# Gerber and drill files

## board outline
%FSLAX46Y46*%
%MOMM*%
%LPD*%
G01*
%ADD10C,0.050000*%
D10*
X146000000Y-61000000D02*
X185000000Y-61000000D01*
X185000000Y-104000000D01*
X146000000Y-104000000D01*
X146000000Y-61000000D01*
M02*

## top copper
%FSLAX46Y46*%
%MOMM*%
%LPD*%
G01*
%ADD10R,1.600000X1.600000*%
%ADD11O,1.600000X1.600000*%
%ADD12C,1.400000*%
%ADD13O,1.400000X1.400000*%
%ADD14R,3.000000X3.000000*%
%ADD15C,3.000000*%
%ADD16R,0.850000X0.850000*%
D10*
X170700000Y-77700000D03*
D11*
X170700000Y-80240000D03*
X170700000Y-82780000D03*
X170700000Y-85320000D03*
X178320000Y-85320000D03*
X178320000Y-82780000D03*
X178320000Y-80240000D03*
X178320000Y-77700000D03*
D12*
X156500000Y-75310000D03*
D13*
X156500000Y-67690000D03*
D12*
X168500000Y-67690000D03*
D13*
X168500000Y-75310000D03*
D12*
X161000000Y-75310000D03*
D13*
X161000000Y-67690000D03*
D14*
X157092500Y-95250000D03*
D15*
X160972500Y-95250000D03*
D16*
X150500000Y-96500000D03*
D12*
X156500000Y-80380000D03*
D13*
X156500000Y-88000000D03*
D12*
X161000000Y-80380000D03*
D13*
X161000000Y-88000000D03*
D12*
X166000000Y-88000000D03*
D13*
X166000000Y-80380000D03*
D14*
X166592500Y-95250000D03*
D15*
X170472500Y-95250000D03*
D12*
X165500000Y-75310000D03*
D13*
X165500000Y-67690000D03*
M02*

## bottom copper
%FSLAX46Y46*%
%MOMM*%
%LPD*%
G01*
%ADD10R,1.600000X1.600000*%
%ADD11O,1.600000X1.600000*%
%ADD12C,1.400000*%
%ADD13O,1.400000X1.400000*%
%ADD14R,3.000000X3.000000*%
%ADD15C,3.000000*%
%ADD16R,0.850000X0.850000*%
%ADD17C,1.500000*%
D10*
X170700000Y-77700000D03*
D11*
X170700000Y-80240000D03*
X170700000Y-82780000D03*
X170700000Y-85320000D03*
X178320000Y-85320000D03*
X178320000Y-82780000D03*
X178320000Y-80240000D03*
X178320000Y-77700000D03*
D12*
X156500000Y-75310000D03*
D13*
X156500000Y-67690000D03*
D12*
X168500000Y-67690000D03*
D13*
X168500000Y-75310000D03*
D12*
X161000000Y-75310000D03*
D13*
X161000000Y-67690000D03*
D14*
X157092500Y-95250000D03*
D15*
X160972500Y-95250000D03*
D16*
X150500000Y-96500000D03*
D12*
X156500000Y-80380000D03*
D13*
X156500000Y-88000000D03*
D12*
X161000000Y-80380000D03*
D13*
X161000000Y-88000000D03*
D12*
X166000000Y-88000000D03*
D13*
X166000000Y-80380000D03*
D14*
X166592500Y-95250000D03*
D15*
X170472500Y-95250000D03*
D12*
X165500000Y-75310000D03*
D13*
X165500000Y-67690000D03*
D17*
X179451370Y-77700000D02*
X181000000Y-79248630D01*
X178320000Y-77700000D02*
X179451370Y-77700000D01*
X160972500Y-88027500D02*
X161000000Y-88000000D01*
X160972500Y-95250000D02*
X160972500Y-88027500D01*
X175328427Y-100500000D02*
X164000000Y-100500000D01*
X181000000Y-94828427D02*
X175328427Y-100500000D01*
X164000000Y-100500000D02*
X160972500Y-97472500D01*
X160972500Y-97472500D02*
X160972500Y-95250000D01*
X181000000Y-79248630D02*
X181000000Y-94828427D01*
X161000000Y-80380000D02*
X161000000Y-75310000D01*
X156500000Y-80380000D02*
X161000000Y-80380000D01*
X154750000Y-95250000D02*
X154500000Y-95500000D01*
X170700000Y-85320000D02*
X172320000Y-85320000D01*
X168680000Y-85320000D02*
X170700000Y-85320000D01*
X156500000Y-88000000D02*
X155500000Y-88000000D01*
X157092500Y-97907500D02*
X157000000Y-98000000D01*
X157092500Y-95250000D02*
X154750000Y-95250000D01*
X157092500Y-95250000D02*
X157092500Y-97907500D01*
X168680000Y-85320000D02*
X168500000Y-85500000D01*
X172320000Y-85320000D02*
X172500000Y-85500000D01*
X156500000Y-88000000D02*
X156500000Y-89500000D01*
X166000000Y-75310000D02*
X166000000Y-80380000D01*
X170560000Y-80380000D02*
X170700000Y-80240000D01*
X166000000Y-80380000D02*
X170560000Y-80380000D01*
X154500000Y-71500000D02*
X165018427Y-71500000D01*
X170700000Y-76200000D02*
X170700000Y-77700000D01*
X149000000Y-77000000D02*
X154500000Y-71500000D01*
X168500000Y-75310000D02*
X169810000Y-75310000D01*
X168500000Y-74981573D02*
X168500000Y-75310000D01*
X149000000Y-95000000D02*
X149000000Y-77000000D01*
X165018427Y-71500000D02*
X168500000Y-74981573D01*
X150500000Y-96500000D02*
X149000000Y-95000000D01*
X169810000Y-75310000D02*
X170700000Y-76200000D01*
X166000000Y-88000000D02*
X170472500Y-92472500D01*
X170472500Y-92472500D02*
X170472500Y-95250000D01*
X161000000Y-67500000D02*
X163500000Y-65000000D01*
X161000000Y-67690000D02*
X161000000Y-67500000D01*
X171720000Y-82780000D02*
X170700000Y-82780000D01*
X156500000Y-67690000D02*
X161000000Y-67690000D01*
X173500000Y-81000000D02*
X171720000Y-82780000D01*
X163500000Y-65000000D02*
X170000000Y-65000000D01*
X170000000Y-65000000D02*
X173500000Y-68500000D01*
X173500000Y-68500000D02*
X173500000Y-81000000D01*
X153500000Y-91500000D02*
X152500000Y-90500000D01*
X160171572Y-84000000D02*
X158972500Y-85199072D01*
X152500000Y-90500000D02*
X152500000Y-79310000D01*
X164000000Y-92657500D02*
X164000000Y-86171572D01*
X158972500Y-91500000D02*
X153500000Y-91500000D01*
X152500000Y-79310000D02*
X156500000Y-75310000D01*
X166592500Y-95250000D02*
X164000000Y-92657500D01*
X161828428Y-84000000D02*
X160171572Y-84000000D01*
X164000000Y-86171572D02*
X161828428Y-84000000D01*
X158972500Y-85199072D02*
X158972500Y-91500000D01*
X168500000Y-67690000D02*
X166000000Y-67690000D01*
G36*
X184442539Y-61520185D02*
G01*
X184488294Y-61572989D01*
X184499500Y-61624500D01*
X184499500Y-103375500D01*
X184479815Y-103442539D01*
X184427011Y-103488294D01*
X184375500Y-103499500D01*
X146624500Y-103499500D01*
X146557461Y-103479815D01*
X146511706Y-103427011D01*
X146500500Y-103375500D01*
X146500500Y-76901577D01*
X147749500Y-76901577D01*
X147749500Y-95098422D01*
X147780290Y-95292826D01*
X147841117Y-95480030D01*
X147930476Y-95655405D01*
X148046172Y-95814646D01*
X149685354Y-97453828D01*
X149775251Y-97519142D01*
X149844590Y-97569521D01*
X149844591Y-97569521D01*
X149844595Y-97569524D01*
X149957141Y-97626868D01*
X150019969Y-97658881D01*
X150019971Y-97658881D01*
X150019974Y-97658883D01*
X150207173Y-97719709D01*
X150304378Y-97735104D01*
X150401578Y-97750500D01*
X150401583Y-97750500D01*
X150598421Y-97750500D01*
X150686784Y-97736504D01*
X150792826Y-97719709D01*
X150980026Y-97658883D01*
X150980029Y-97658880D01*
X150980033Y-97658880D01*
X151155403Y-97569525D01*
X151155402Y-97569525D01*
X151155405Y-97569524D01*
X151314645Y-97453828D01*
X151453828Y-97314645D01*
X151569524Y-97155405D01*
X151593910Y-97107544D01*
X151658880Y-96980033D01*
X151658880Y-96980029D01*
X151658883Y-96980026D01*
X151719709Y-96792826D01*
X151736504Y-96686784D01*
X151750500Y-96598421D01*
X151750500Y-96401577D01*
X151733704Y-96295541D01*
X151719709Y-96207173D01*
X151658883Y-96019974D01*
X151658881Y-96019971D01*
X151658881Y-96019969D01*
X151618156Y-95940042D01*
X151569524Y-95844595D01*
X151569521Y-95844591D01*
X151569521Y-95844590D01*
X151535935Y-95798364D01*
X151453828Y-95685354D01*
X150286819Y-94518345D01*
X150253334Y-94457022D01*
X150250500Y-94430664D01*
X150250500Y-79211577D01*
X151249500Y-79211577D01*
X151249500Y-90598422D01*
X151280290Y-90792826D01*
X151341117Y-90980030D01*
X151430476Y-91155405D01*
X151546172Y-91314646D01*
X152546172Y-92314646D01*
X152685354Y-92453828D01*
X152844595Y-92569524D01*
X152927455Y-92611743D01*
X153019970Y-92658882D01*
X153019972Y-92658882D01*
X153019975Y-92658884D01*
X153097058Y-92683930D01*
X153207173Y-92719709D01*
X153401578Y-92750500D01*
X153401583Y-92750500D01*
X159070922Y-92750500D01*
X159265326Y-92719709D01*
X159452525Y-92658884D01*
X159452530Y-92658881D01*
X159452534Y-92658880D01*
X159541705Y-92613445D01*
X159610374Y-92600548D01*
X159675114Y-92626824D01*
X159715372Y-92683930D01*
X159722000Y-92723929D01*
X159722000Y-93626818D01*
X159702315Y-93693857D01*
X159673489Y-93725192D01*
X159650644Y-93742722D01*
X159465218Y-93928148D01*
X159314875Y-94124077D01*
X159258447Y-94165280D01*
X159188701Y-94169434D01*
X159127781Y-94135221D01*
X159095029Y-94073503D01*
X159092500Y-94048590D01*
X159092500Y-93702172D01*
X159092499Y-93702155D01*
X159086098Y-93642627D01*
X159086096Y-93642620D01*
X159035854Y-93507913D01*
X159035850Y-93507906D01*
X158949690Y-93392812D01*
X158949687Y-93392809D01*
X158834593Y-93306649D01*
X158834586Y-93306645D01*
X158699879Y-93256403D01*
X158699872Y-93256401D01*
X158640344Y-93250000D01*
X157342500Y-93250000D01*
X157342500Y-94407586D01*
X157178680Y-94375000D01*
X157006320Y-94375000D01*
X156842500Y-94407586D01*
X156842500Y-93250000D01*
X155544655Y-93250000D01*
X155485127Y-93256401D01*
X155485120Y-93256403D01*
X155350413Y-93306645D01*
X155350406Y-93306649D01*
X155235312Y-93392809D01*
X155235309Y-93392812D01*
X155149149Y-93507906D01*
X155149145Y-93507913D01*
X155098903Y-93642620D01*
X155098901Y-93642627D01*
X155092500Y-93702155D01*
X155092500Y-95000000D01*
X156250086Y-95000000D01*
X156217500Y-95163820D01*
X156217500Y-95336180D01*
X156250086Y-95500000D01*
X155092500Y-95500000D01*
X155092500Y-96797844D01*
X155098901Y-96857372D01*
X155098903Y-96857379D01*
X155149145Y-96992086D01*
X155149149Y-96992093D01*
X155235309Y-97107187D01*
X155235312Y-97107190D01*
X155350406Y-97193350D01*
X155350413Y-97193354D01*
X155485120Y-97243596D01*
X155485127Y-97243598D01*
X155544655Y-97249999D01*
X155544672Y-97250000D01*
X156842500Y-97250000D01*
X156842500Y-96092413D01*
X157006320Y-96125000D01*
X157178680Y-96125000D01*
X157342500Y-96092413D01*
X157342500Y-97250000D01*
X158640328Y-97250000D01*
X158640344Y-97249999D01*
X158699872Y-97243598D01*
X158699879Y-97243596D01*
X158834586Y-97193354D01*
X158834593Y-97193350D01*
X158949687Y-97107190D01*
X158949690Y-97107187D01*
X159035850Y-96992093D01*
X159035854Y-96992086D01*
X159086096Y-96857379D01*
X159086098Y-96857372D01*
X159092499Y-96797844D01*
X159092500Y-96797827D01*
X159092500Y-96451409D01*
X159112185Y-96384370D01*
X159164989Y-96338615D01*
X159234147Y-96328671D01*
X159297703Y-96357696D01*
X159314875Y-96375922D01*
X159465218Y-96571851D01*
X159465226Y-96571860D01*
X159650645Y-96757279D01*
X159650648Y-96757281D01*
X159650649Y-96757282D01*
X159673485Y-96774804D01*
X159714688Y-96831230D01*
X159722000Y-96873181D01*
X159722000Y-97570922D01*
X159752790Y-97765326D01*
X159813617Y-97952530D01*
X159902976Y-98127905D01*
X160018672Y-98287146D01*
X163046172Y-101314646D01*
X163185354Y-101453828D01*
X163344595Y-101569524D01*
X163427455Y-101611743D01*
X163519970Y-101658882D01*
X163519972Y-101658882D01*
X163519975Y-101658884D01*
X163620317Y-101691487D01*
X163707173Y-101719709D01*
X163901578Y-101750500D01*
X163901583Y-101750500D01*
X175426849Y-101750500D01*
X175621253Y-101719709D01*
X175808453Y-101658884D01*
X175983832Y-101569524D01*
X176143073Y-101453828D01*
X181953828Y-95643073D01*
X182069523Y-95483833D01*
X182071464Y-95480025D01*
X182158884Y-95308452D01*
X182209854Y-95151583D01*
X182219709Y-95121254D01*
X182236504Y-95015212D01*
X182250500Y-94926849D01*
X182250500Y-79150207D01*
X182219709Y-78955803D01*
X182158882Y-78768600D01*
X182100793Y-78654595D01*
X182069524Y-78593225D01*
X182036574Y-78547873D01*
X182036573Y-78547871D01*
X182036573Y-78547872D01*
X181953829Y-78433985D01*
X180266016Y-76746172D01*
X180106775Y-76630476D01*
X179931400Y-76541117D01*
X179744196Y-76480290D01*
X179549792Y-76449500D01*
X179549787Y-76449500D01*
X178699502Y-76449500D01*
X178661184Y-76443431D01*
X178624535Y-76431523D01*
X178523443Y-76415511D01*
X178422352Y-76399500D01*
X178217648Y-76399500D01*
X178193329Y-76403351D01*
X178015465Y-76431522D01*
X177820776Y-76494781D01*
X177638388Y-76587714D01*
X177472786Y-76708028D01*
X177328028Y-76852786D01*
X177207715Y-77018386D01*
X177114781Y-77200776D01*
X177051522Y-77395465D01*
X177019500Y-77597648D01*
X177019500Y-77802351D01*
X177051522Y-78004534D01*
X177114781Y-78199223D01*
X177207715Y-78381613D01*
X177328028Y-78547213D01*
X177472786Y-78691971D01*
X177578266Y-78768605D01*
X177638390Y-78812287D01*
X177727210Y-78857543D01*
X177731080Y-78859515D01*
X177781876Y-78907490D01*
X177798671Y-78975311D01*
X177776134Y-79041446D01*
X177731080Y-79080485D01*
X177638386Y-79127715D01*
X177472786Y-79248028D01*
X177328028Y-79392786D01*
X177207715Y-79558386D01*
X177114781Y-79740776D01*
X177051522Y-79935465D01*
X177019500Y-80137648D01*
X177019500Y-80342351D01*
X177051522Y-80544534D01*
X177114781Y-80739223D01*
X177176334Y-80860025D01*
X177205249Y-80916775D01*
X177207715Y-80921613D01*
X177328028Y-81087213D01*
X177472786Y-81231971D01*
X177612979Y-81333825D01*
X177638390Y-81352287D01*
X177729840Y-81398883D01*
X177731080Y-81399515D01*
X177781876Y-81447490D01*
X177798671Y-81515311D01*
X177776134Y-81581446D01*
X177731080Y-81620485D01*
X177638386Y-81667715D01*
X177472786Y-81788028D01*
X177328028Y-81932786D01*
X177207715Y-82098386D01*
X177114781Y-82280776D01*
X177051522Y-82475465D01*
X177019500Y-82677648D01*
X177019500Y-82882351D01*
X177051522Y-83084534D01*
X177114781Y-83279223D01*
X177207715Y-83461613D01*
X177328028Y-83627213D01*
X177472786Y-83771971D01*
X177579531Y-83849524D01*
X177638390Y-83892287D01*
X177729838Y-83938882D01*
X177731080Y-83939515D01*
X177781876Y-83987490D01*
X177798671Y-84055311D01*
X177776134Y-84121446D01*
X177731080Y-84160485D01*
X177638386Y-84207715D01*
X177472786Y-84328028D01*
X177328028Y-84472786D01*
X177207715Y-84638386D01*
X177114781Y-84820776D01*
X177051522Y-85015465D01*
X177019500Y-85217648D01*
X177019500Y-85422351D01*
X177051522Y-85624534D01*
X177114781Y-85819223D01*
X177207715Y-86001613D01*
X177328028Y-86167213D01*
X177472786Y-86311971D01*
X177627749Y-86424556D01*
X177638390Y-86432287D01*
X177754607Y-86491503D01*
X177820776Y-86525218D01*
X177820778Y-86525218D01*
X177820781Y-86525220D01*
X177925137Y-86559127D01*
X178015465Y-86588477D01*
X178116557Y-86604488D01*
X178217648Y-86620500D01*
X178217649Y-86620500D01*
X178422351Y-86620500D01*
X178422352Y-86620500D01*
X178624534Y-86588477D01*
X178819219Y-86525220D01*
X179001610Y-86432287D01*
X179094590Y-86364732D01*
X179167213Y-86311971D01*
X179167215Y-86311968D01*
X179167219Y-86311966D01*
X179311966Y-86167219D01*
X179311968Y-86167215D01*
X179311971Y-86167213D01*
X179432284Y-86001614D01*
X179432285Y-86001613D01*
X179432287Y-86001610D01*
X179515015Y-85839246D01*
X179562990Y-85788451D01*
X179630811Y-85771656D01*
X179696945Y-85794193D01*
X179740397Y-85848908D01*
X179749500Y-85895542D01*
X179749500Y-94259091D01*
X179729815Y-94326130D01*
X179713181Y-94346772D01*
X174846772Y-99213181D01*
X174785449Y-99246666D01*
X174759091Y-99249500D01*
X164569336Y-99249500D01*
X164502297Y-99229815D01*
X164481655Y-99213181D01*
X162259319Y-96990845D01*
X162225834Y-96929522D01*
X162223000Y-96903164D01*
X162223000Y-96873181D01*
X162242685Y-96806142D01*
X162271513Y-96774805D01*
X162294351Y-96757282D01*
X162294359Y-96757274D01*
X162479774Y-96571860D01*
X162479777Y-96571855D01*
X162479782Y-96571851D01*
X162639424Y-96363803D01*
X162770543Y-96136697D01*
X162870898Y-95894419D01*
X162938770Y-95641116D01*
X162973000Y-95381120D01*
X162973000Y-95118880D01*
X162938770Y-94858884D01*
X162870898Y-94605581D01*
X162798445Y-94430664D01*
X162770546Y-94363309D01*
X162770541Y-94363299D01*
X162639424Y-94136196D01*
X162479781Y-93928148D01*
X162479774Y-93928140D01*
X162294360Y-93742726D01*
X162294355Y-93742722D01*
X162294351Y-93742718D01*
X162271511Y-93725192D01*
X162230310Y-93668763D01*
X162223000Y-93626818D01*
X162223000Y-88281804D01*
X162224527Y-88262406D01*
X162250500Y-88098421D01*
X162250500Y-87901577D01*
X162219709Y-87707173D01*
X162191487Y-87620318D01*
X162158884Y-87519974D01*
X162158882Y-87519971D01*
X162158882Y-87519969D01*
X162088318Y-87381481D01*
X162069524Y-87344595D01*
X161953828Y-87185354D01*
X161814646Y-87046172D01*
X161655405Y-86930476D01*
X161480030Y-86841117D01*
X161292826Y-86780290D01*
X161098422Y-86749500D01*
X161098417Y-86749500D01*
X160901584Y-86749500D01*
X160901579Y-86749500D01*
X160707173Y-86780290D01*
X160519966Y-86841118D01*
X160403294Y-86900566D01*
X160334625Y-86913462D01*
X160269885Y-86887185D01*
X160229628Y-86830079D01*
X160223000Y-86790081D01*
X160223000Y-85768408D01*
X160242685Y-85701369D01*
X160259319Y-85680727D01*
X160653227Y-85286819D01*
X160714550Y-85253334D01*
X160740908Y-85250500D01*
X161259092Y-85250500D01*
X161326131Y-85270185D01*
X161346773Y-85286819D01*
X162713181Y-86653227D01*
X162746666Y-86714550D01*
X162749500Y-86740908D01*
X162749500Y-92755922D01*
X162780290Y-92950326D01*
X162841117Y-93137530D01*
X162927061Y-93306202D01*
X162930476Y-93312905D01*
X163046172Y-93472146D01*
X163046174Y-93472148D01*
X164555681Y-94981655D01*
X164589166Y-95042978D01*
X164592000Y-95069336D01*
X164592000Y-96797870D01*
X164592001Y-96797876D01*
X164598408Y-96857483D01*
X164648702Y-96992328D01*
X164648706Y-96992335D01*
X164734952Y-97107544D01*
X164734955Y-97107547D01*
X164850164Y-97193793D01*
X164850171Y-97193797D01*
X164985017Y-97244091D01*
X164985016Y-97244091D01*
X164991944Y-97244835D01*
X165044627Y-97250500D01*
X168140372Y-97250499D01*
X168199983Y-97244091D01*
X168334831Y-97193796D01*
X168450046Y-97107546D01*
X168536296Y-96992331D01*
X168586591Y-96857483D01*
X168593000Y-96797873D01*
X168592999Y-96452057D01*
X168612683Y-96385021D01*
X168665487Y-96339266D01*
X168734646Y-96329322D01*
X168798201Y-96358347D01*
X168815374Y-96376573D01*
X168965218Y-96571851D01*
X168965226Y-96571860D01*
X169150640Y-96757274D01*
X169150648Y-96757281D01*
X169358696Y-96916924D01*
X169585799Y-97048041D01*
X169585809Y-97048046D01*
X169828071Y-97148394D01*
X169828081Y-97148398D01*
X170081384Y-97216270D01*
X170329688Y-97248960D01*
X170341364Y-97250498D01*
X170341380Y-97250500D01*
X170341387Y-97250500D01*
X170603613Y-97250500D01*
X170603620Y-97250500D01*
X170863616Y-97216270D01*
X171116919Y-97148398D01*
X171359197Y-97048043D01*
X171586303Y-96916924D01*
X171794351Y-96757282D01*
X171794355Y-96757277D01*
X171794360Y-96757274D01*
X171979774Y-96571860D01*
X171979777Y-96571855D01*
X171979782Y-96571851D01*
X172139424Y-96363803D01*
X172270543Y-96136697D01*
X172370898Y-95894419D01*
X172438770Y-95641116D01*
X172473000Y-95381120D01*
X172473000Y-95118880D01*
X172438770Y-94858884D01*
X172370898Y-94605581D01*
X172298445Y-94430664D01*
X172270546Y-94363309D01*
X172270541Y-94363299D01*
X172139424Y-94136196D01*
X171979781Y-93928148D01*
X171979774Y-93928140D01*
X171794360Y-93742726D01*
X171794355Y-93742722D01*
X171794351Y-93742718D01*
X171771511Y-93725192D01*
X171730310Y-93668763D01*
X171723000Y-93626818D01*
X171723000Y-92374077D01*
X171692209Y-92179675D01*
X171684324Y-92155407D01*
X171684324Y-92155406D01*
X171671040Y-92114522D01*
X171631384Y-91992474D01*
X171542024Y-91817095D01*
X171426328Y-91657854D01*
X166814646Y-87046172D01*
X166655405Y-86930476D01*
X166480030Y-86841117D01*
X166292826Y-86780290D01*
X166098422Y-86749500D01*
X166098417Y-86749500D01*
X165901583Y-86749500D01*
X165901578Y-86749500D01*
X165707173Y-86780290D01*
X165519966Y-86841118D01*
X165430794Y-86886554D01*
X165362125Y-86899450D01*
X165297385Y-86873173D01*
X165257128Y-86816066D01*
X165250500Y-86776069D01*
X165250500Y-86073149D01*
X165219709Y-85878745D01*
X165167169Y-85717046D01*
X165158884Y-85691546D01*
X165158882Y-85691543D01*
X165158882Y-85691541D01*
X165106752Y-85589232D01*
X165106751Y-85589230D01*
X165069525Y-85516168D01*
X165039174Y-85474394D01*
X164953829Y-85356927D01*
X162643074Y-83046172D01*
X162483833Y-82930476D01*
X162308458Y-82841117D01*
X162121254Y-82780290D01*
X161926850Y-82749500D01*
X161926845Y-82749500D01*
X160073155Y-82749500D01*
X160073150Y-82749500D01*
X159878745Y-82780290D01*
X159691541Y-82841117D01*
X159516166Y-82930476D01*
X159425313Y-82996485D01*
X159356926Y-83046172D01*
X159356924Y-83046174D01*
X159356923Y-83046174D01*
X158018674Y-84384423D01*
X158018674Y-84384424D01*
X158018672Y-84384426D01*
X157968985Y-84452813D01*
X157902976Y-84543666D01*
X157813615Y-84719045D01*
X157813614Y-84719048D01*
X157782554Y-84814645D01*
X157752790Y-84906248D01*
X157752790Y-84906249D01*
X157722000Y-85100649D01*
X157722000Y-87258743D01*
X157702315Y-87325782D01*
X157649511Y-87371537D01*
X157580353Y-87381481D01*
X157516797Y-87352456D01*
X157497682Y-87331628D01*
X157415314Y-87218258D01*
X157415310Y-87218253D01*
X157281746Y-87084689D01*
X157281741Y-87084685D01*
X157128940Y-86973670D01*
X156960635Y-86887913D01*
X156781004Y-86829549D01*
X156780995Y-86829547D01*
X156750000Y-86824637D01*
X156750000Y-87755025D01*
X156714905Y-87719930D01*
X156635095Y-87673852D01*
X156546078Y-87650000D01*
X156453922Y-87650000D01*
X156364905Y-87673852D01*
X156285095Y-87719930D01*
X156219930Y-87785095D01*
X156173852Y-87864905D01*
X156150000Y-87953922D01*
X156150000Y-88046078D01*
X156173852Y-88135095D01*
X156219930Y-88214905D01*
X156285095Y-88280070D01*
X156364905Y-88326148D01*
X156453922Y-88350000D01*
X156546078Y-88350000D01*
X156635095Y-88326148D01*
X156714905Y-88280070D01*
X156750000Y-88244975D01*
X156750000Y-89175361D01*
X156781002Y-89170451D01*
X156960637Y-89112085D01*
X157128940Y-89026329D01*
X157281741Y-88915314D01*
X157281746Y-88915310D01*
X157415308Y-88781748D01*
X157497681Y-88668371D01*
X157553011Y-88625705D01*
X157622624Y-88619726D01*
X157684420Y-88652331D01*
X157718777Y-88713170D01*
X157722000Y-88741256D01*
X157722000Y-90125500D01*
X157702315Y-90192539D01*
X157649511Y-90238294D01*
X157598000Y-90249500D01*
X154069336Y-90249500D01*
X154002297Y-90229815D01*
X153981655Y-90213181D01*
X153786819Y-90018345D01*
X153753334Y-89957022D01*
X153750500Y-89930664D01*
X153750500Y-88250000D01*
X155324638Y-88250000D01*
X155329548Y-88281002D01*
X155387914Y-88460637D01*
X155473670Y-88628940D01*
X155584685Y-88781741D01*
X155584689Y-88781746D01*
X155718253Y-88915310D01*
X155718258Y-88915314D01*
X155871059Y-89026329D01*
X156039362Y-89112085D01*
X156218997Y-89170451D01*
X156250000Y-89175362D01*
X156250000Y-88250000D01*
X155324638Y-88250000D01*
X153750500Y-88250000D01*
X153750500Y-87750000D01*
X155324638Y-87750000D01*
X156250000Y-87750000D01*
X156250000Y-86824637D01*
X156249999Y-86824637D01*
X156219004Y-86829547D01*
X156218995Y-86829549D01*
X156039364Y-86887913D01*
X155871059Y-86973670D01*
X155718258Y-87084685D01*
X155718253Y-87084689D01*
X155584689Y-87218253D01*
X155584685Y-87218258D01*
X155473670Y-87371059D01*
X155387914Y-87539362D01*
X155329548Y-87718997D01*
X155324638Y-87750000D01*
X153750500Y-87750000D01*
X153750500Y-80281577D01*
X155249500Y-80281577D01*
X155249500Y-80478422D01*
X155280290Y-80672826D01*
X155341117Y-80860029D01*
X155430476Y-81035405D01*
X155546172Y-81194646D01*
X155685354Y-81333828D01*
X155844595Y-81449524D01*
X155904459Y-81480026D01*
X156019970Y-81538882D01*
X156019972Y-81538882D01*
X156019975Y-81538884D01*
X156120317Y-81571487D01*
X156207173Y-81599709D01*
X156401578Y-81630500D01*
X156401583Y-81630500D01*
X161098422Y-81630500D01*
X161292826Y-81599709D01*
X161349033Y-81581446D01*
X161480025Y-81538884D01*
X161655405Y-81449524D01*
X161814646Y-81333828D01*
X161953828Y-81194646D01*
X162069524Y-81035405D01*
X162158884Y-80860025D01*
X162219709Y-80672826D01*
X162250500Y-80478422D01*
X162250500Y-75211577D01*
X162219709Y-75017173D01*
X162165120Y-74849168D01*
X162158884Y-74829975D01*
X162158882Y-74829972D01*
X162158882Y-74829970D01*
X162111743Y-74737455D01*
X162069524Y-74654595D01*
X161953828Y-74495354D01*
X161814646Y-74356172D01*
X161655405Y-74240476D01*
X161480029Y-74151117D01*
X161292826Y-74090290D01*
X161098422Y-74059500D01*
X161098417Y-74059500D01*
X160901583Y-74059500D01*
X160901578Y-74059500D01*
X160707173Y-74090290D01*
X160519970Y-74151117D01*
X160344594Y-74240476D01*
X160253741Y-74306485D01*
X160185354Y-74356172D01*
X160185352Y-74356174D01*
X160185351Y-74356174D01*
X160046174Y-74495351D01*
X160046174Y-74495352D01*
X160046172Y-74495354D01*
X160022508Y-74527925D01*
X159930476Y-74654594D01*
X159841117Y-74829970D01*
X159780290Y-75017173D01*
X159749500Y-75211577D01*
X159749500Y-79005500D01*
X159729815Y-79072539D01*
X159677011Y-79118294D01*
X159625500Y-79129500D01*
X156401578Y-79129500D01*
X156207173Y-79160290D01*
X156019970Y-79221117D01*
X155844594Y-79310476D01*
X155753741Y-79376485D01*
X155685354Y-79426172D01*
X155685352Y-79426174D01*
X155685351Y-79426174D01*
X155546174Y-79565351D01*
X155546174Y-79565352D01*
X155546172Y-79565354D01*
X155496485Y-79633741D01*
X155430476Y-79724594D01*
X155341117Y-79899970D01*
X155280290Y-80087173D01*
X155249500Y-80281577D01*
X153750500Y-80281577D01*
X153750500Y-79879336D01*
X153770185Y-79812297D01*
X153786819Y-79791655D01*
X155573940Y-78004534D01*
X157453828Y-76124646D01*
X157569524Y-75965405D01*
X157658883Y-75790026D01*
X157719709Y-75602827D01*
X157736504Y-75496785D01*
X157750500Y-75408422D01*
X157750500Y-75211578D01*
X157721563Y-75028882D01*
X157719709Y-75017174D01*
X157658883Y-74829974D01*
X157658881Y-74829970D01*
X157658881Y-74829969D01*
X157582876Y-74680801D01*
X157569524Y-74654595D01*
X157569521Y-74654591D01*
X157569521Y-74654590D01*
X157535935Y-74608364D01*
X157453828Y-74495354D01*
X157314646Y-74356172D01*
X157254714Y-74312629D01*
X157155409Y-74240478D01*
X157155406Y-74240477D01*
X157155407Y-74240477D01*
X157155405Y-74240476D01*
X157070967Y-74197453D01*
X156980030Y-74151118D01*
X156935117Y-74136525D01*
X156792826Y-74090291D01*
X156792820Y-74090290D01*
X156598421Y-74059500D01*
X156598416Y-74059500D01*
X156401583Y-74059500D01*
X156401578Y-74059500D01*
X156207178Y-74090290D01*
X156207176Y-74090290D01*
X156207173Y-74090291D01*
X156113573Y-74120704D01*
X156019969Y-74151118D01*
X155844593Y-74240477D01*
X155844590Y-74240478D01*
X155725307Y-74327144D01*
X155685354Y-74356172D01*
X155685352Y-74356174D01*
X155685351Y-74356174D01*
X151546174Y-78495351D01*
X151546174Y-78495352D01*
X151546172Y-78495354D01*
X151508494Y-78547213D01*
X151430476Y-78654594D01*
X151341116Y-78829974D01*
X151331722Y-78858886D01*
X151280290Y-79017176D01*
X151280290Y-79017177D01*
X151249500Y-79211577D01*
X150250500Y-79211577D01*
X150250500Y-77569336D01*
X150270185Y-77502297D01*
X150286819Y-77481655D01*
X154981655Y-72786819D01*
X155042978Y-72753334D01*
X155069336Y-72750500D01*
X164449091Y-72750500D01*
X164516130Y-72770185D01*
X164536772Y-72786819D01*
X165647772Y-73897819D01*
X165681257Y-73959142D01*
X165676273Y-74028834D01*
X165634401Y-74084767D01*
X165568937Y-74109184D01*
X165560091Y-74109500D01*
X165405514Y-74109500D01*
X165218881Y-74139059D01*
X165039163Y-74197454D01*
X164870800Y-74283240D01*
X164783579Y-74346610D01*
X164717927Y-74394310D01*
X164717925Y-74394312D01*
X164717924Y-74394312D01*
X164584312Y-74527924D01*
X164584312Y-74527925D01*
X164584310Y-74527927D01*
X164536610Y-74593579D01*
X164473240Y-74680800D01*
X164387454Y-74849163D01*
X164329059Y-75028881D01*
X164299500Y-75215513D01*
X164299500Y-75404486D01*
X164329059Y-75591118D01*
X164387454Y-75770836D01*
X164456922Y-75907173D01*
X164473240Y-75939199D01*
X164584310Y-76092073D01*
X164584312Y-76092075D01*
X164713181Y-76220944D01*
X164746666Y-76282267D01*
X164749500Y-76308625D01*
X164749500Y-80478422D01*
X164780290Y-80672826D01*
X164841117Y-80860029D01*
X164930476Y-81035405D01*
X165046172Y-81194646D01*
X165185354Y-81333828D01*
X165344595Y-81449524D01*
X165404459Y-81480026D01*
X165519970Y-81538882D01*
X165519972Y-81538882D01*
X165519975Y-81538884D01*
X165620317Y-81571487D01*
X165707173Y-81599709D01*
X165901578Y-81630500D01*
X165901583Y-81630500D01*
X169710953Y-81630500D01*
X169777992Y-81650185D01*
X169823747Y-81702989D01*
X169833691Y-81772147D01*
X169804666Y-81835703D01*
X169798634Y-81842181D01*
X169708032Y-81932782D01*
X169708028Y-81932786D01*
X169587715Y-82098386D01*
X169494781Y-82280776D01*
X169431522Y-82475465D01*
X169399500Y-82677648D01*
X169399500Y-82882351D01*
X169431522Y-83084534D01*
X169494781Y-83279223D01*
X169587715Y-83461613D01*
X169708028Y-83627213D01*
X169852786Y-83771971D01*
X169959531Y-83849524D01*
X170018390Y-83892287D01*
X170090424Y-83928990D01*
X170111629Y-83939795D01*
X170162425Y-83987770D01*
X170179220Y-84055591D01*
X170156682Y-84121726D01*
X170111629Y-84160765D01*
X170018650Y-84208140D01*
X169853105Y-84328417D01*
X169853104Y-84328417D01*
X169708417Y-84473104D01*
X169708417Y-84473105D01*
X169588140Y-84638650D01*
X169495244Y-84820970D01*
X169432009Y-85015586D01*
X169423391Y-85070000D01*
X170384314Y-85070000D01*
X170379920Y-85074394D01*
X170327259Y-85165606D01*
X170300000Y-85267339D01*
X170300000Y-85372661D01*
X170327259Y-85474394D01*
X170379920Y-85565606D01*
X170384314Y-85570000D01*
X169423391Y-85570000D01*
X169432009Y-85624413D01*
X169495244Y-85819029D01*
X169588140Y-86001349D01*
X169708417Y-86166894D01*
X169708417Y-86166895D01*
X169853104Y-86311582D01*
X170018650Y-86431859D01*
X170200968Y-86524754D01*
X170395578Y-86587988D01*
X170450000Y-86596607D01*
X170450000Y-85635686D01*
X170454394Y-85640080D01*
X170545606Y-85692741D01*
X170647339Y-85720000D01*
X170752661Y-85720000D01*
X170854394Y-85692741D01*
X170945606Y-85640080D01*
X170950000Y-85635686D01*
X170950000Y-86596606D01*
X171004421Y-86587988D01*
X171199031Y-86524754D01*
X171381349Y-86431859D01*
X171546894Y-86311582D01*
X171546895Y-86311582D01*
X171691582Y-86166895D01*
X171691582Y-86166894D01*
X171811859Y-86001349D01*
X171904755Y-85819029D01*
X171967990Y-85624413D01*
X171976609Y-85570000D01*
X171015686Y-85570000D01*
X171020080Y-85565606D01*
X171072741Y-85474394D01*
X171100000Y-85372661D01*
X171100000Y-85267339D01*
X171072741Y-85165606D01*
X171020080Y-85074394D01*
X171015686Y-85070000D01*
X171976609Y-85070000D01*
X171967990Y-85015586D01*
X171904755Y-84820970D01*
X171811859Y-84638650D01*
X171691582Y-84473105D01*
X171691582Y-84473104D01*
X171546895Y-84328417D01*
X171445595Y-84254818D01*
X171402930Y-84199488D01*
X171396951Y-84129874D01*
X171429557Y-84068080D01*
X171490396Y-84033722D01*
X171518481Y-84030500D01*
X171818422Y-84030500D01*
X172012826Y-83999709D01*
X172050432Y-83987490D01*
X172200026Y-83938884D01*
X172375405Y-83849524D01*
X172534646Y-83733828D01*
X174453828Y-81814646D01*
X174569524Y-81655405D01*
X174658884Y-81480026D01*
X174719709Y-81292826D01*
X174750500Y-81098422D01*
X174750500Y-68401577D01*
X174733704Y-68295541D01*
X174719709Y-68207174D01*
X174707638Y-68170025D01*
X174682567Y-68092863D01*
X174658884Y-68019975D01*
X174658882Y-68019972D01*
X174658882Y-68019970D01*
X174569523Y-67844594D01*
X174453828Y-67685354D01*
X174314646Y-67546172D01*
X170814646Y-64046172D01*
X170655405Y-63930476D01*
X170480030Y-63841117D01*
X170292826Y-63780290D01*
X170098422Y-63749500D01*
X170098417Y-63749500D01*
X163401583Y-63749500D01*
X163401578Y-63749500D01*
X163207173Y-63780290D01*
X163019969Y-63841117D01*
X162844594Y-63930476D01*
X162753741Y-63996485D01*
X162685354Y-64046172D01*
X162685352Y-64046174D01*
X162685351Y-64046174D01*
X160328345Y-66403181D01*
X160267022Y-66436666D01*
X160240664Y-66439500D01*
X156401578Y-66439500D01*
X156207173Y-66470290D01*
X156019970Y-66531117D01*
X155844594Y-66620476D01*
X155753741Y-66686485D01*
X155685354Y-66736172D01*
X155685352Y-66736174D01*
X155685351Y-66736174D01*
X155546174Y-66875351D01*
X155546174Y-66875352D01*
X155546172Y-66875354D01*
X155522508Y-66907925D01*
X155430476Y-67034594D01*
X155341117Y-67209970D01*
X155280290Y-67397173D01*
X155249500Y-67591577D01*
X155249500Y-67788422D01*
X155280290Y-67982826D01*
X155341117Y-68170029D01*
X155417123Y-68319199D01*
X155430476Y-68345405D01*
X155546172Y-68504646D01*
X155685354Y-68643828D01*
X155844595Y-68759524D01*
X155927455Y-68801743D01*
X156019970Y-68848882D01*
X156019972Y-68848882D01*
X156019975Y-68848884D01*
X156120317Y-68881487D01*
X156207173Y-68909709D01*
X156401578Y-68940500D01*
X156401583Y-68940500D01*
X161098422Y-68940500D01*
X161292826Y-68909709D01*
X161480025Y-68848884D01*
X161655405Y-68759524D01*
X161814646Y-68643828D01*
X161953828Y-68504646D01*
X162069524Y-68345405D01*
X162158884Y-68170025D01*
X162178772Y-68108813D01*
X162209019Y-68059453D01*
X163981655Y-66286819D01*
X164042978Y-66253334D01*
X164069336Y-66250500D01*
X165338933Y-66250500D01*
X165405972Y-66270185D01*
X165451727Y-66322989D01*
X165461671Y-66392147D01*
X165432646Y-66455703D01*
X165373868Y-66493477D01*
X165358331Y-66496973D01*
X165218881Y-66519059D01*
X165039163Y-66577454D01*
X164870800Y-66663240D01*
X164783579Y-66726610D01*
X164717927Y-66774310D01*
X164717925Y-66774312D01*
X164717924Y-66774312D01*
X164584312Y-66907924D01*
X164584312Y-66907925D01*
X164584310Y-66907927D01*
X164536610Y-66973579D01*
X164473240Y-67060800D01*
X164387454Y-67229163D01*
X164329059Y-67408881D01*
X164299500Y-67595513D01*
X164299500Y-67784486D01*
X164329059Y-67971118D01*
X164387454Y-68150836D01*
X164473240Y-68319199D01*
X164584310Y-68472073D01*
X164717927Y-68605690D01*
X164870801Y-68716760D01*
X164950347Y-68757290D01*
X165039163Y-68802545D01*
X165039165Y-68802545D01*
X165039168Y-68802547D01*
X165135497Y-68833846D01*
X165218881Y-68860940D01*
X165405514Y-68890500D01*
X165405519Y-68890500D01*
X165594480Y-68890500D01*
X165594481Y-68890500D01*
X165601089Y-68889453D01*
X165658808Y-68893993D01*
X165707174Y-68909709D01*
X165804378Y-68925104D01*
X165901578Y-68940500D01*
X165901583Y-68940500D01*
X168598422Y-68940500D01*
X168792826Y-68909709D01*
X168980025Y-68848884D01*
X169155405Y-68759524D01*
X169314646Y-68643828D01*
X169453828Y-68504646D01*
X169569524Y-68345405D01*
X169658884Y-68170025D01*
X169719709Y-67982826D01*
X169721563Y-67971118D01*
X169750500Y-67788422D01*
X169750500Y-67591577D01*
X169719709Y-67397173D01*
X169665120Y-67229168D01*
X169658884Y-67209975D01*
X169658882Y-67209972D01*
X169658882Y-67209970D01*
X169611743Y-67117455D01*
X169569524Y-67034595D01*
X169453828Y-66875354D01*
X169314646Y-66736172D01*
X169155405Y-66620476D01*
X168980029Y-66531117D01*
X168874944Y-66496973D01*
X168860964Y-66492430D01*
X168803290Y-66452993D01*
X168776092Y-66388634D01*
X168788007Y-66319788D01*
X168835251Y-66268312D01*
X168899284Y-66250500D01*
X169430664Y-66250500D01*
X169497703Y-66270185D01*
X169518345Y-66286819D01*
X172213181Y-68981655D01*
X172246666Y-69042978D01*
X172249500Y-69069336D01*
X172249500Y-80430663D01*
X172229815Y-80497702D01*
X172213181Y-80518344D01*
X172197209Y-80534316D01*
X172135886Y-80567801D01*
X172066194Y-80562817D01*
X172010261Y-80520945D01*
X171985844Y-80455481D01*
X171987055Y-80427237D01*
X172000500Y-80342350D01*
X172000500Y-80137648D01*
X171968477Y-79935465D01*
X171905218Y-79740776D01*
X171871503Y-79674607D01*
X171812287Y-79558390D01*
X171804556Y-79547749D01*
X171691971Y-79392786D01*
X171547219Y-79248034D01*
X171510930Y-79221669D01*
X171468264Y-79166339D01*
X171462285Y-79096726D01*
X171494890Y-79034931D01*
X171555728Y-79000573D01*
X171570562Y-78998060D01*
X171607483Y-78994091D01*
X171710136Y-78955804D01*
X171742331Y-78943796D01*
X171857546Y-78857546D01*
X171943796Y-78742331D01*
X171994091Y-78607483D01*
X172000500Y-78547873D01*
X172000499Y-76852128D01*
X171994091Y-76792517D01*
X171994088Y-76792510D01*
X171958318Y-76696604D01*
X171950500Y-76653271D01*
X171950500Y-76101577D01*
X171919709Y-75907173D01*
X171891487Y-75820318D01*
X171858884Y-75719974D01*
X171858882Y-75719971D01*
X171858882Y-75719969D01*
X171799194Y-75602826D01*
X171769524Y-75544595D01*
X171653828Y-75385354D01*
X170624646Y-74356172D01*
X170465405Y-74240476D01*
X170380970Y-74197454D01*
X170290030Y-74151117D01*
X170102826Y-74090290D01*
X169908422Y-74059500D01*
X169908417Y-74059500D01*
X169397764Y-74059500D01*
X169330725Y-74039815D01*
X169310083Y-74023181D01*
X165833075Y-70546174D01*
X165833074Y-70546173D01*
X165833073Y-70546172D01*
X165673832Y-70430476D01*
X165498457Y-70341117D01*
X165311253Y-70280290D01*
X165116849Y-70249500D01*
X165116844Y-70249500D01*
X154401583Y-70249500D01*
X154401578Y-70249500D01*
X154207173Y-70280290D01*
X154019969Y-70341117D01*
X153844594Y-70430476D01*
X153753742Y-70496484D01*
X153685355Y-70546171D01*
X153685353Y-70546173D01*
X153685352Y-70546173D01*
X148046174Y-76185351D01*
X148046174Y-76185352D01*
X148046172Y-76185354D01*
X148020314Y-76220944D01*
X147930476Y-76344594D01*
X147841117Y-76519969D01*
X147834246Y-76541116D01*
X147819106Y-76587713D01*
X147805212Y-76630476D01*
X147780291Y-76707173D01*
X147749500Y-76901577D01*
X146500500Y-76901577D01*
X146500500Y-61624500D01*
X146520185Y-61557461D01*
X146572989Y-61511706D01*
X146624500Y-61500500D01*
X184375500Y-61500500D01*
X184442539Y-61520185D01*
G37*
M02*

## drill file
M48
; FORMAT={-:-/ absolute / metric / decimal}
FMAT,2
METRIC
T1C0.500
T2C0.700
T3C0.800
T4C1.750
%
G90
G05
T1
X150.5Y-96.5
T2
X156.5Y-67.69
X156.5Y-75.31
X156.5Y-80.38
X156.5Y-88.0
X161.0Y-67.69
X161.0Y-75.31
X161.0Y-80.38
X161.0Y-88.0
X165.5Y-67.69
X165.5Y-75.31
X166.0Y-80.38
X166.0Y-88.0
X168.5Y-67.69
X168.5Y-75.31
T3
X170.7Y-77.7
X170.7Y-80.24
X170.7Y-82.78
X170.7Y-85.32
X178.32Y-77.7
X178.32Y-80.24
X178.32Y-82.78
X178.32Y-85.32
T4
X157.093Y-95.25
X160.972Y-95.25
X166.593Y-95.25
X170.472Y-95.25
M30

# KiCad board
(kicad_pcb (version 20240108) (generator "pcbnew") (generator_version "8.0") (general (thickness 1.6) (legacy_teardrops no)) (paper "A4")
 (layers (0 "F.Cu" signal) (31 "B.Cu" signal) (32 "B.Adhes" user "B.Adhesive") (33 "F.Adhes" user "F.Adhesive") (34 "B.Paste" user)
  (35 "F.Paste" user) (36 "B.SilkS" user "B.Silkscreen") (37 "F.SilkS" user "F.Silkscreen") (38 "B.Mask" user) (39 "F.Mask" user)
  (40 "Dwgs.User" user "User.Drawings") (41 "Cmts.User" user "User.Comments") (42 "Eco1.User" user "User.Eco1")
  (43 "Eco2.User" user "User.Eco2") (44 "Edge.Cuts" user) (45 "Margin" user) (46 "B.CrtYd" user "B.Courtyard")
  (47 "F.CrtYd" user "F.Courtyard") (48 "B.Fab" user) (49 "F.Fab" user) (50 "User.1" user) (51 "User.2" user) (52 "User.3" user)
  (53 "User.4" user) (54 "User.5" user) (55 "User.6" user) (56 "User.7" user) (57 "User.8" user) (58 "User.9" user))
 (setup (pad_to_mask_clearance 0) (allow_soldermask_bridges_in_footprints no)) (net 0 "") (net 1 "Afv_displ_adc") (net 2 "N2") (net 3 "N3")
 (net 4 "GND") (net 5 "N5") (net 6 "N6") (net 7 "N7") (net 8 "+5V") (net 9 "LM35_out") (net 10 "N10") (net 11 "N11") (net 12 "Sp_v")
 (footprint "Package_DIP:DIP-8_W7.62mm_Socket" (layer "F.Cu") (at 170.7 77.7)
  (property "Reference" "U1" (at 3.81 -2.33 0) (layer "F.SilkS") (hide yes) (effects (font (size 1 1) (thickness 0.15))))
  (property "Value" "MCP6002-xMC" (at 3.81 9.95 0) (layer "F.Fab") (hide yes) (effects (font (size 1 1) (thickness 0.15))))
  (pad "1" thru_hole rect (at 0 0) (size 1.6 1.6) (drill 0.8) (layers "*.Cu" "*.Mask") (remove_unused_layers no) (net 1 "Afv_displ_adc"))
  (pad "2" thru_hole oval (at 0 2.54) (size 1.6 1.6) (drill 0.8) (layers "*.Cu" "*.Mask") (remove_unused_layers no) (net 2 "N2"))
  (pad "3" thru_hole oval (at 0 5.08) (size 1.6 1.6) (drill 0.8) (layers "*.Cu" "*.Mask") (remove_unused_layers no) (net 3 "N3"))
  (pad "4" thru_hole oval (at 0 7.62) (size 1.6 1.6) (drill 0.8) (layers "*.Cu" "*.Mask") (remove_unused_layers no) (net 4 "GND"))
  (pad "5" thru_hole oval (at 7.62 7.62) (size 1.6 1.6) (drill 0.8) (layers "*.Cu" "*.Mask") (remove_unused_layers no) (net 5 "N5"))
  (pad "6" thru_hole oval (at 7.62 5.08) (size 1.6 1.6) (drill 0.8) (layers "*.Cu" "*.Mask") (remove_unused_layers no) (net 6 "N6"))
  (pad "7" thru_hole oval (at 7.62 2.54) (size 1.6 1.6) (drill 0.8) (layers "*.Cu" "*.Mask") (remove_unused_layers no) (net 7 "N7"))
  (pad "8" thru_hole oval (at 7.62 0) (size 1.6 1.6) (drill 0.8) (layers "*.Cu" "*.Mask") (remove_unused_layers no) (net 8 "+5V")))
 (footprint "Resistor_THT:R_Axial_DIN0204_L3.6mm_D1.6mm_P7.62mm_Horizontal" (layer "F.Cu") (at 156.5 75.31 90)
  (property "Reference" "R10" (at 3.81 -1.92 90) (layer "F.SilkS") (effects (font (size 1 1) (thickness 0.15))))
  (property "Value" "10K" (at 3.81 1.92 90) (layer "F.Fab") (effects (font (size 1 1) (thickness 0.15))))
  (pad "1" thru_hole circle (at 0 0 90) (size 1.4 1.4) (drill 0.7) (layers "*.Cu" "*.Mask") (remove_unused_layers no) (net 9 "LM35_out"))
  (pad "2" thru_hole oval (at 7.62 0 90) (size 1.4 1.4) (drill 0.7) (layers "*.Cu" "*.Mask") (remove_unused_layers no) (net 3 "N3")))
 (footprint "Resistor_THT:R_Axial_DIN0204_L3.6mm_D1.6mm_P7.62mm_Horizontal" (layer "F.Cu") (at 168.5 67.69 -90)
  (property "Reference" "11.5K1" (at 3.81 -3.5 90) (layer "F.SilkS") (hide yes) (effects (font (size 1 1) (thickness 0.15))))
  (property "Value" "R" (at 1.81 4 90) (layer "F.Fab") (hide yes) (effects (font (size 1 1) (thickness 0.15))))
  (pad "1" thru_hole circle (at 0 0 270) (size 1.4 1.4) (drill 0.7) (layers "*.Cu" "*.Mask") (remove_unused_layers no) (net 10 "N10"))
  (pad "2" thru_hole oval (at 7.62 0 270) (size 1.4 1.4) (drill 0.7) (layers "*.Cu" "*.Mask") (remove_unused_layers no)
   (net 1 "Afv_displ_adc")))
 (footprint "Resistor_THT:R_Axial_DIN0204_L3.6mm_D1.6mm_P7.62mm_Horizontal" (layer "F.Cu") (at 161 75.31 90)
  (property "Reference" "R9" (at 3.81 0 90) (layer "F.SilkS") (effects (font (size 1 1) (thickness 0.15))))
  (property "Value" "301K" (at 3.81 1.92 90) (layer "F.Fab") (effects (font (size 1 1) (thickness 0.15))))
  (pad "1" thru_hole circle (at 0 0 90) (size 1.4 1.4) (drill 0.7) (layers "*.Cu" "*.Mask") (remove_unused_layers no) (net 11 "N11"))
  (pad "2" thru_hole oval (at 7.62 0 90) (size 1.4 1.4) (drill 0.7) (layers "*.Cu" "*.Mask") (remove_unused_layers no) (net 3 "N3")))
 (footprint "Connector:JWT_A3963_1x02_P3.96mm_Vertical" (layer "F.Cu") (at 157.0925 95.25)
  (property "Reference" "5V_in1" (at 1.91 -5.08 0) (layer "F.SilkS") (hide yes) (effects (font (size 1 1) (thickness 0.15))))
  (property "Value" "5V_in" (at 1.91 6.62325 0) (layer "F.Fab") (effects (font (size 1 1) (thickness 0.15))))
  (pad "1" thru_hole rect (at 0 0) (size 3 3) (drill 1.75) (layers "*.Cu" "*.Mask") (remove_unused_layers no) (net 4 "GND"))
  (pad "2" thru_hole circle (at 3.88 0) (size 3 3) (drill 1.75) (layers "*.Cu" "*.Mask") (remove_unused_layers no) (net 8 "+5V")))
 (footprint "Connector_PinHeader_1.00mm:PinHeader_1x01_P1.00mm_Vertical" (layer "F.Cu") (at 150.5 96.5)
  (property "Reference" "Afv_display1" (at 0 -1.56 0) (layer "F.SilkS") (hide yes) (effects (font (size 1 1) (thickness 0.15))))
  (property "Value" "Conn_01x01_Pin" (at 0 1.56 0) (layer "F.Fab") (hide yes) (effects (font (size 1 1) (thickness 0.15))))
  (pad "1" thru_hole rect (at 0 0) (size 0.85 0.85) (drill 0.5) (layers "*.Cu" "*.Mask") (remove_unused_layers no) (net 1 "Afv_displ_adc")))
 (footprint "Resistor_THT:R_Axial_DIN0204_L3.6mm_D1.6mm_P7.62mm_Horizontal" (layer "F.Cu") (at 156.5 80.38 -90)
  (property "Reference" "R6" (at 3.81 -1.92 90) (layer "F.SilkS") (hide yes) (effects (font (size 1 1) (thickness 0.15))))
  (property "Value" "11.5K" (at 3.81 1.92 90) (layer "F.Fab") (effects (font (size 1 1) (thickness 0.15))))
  (pad "1" thru_hole circle (at 0 0 270) (size 1.4 1.4) (drill 0.7) (layers "*.Cu" "*.Mask") (remove_unused_layers no) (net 11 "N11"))
  (pad "2" thru_hole oval (at 7.62 0 270) (size 1.4 1.4) (drill 0.7) (layers "*.Cu" "*.Mask") (remove_unused_layers no) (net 4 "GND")))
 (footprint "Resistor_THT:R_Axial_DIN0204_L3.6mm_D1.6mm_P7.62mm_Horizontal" (layer "F.Cu") (at 161 80.38 -90)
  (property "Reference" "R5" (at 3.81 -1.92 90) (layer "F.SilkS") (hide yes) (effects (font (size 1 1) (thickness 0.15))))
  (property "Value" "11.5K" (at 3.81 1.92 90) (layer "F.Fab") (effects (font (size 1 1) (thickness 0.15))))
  (pad "1" thru_hole circle (at 0 0 270) (size 1.4 1.4) (drill 0.7) (layers "*.Cu" "*.Mask") (remove_unused_layers no) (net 11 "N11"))
  (pad "2" thru_hole oval (at 7.62 0 270) (size 1.4 1.4) (drill 0.7) (layers "*.Cu" "*.Mask") (remove_unused_layers no) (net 8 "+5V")))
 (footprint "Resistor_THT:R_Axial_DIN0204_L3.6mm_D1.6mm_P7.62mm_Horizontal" (layer "F.Cu") (at 166 88 90)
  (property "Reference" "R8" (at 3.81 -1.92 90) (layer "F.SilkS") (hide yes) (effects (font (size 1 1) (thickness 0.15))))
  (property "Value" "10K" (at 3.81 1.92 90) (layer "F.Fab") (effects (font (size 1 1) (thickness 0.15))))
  (pad "1" thru_hole circle (at 0 0 90) (size 1.4 1.4) (drill 0.7) (layers "*.Cu" "*.Mask") (remove_unused_layers no) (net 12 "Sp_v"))
  (pad "2" thru_hole oval (at 7.62 0 90) (size 1.4 1.4) (drill 0.7) (layers "*.Cu" "*.Mask") (remove_unused_layers no) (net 2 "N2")))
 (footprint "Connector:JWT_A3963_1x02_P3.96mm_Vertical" (layer "F.Cu") (at 166.5925 95.25)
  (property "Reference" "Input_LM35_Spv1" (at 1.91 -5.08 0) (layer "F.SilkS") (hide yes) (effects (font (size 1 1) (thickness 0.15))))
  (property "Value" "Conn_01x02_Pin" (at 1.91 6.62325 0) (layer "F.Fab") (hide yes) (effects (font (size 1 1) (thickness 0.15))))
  (pad "1" thru_hole rect (at 0 0) (size 3 3) (drill 1.75) (layers "*.Cu" "*.Mask") (remove_unused_layers no) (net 9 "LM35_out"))
  (pad "2" thru_hole circle (at 3.88 0) (size 3 3) (drill 1.75) (layers "*.Cu" "*.Mask") (remove_unused_layers no) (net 12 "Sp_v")))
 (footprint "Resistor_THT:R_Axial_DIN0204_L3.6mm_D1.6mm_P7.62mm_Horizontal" (layer "F.Cu") (at 165.5 75.31 90)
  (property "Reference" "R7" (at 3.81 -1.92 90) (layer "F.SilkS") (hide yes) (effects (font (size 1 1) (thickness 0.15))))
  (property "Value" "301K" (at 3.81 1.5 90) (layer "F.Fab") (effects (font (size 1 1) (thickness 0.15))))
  (pad "1" thru_hole circle (at 0 0 90) (size 1.4 1.4) (drill 0.7) (layers "*.Cu" "*.Mask") (remove_unused_layers no) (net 2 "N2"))
  (pad "2" thru_hole oval (at 7.62 0 90) (size 1.4 1.4) (drill 0.7) (layers "*.Cu" "*.Mask") (remove_unused_layers no) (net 10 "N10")))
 (gr_rect (start 146 61) (end 185 104) (stroke (width 0.05) (type default)) (fill none) (layer "Edge.Cuts"))
 (segment (start 179.45137 77.7) (end 181 79.24863) (width 1.5) (layer "B.Cu") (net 8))
 (segment (start 178.32 77.7) (end 179.45137 77.7) (width 1.5) (layer "B.Cu") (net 8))
 (segment (start 160.9725 88.0275) (end 161 88) (width 1.5) (layer "B.Cu") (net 8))
 (segment (start 160.9725 95.25) (end 160.9725 88.0275) (width 1.5) (layer "B.Cu") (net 8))
 (segment (start 175.328427 100.5) (end 164 100.5) (width 1.5) (layer "B.Cu") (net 8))
 (segment (start 181 94.828427) (end 175.328427 100.5) (width 1.5) (layer "B.Cu") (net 8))
 (segment (start 164 100.5) (end 160.9725 97.4725) (width 1.5) (layer "B.Cu") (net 8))
 (segment (start 160.9725 97.4725) (end 160.9725 95.25) (width 1.5) (layer "B.Cu") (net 8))
 (segment (start 181 79.24863) (end 181 94.828427) (width 1.5) (layer "B.Cu") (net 8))
 (segment (start 161 80.38) (end 161 75.31) (width 1.5) (layer "B.Cu") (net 11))
 (segment (start 156.5 80.38) (end 161 80.38) (width 1.5) (layer "B.Cu") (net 11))
 (segment (start 154.75 95.25) (end 154.5 95.5) (width 1.5) (layer "B.Cu") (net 4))
 (segment (start 170.7 85.32) (end 172.32 85.32) (width 1.5) (layer "B.Cu") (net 4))
 (segment (start 168.68 85.32) (end 170.7 85.32) (width 1.5) (layer "B.Cu") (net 4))
 (segment (start 156.5 88) (end 155.5 88) (width 1.5) (layer "B.Cu") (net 4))
 (segment (start 157.0925 97.9075) (end 157 98) (width 1.5) (layer "B.Cu") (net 4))
 (segment (start 157.0925 95.25) (end 154.75 95.25) (width 1.5) (layer "B.Cu") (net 4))
 (segment (start 157.0925 95.25) (end 157.0925 97.9075) (width 1.5) (layer "B.Cu") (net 4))
 (segment (start 168.68 85.32) (end 168.5 85.5) (width 1.5) (layer "B.Cu") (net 4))
 (segment (start 172.32 85.32) (end 172.5 85.5) (width 1.5) (layer "B.Cu") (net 4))
 (segment (start 156.5 88) (end 156.5 89.5) (width 1.5) (layer "B.Cu") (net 4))
 (segment (start 166 75.31) (end 166 80.38) (width 1.5) (layer "B.Cu") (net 2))
 (segment (start 170.56 80.38) (end 170.7 80.24) (width 1.5) (layer "B.Cu") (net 2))
 (segment (start 166 80.38) (end 170.56 80.38) (width 1.5) (layer "B.Cu") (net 2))
 (segment (start 154.5 71.5) (end 165.018427 71.5) (width 1.5) (layer "B.Cu") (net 1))
 (segment (start 170.7 76.2) (end 170.7 77.7) (width 1.5) (layer "B.Cu") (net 1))
 (segment (start 149 77) (end 154.5 71.5) (width 1.5) (layer "B.Cu") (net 1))
 (segment (start 168.5 75.31) (end 169.81 75.31) (width 1.5) (layer "B.Cu") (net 1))
 (segment (start 168.5 74.981573) (end 168.5 75.31) (width 1.5) (layer "B.Cu") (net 1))
 (segment (start 149 95) (end 149 77) (width 1.5) (layer "B.Cu") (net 1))
 (segment (start 165.018427 71.5) (end 168.5 74.981573) (width 1.5) (layer "B.Cu") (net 1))
 (segment (start 150.5 96.5) (end 149 95) (width 1.5) (layer "B.Cu") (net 1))
 (segment (start 169.81 75.31) (end 170.7 76.2) (width 1.5) (layer "B.Cu") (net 1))
 (segment (start 166 88) (end 170.4725 92.4725) (width 1.5) (layer "B.Cu") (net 12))
 (segment (start 170.4725 92.4725) (end 170.4725 95.25) (width 1.5) (layer "B.Cu") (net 12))
 (segment (start 161 67.5) (end 163.5 65) (width 1.5) (layer "B.Cu") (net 3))
 (segment (start 161 67.69) (end 161 67.5) (width 1.5) (layer "B.Cu") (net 3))
 (segment (start 171.72 82.78) (end 170.7 82.78) (width 1.5) (layer "B.Cu") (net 3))
 (segment (start 156.5 67.69) (end 161 67.69) (width 1.5) (layer "B.Cu") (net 3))
 (segment (start 173.5 81) (end 171.72 82.78) (width 1.5) (layer "B.Cu") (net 3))
 (segment (start 163.5 65) (end 170 65) (width 1.5) (layer "B.Cu") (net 3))
 (segment (start 170 65) (end 173.5 68.5) (width 1.5) (layer "B.Cu") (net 3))
 (segment (start 173.5 68.5) (end 173.5 81) (width 1.5) (layer "B.Cu") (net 3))
 (segment (start 153.5 91.5) (end 152.5 90.5) (width 1.5) (layer "B.Cu") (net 9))
 (segment (start 160.171572 84) (end 158.9725 85.199072) (width 1.5) (layer "B.Cu") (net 9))
 (segment (start 152.5 90.5) (end 152.5 79.31) (width 1.5) (layer "B.Cu") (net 9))
 (segment (start 164 92.6575) (end 164 86.171572) (width 1.5) (layer "B.Cu") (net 9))
 (segment (start 158.9725 91.5) (end 153.5 91.5) (width 1.5) (layer "B.Cu") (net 9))
 (segment (start 152.5 79.31) (end 156.5 75.31) (width 1.5) (layer "B.Cu") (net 9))
 (segment (start 166.5925 95.25) (end 164 92.6575) (width 1.5) (layer "B.Cu") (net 9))
 (segment (start 161.828428 84) (end 160.171572 84) (width 1.5) (layer "B.Cu") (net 9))
 (segment (start 164 86.171572) (end 161.828428 84) (width 1.5) (layer "B.Cu") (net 9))
 (segment (start 158.9725 85.199072) (end 158.9725 91.5) (width 1.5) (layer "B.Cu") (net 9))
 (segment (start 168.5 67.69) (end 166 67.69) (width 1.5) (layer "B.Cu") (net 10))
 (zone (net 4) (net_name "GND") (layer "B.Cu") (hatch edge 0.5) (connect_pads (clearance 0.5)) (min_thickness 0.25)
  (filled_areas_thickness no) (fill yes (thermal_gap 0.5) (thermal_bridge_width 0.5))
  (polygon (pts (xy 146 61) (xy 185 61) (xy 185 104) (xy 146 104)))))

